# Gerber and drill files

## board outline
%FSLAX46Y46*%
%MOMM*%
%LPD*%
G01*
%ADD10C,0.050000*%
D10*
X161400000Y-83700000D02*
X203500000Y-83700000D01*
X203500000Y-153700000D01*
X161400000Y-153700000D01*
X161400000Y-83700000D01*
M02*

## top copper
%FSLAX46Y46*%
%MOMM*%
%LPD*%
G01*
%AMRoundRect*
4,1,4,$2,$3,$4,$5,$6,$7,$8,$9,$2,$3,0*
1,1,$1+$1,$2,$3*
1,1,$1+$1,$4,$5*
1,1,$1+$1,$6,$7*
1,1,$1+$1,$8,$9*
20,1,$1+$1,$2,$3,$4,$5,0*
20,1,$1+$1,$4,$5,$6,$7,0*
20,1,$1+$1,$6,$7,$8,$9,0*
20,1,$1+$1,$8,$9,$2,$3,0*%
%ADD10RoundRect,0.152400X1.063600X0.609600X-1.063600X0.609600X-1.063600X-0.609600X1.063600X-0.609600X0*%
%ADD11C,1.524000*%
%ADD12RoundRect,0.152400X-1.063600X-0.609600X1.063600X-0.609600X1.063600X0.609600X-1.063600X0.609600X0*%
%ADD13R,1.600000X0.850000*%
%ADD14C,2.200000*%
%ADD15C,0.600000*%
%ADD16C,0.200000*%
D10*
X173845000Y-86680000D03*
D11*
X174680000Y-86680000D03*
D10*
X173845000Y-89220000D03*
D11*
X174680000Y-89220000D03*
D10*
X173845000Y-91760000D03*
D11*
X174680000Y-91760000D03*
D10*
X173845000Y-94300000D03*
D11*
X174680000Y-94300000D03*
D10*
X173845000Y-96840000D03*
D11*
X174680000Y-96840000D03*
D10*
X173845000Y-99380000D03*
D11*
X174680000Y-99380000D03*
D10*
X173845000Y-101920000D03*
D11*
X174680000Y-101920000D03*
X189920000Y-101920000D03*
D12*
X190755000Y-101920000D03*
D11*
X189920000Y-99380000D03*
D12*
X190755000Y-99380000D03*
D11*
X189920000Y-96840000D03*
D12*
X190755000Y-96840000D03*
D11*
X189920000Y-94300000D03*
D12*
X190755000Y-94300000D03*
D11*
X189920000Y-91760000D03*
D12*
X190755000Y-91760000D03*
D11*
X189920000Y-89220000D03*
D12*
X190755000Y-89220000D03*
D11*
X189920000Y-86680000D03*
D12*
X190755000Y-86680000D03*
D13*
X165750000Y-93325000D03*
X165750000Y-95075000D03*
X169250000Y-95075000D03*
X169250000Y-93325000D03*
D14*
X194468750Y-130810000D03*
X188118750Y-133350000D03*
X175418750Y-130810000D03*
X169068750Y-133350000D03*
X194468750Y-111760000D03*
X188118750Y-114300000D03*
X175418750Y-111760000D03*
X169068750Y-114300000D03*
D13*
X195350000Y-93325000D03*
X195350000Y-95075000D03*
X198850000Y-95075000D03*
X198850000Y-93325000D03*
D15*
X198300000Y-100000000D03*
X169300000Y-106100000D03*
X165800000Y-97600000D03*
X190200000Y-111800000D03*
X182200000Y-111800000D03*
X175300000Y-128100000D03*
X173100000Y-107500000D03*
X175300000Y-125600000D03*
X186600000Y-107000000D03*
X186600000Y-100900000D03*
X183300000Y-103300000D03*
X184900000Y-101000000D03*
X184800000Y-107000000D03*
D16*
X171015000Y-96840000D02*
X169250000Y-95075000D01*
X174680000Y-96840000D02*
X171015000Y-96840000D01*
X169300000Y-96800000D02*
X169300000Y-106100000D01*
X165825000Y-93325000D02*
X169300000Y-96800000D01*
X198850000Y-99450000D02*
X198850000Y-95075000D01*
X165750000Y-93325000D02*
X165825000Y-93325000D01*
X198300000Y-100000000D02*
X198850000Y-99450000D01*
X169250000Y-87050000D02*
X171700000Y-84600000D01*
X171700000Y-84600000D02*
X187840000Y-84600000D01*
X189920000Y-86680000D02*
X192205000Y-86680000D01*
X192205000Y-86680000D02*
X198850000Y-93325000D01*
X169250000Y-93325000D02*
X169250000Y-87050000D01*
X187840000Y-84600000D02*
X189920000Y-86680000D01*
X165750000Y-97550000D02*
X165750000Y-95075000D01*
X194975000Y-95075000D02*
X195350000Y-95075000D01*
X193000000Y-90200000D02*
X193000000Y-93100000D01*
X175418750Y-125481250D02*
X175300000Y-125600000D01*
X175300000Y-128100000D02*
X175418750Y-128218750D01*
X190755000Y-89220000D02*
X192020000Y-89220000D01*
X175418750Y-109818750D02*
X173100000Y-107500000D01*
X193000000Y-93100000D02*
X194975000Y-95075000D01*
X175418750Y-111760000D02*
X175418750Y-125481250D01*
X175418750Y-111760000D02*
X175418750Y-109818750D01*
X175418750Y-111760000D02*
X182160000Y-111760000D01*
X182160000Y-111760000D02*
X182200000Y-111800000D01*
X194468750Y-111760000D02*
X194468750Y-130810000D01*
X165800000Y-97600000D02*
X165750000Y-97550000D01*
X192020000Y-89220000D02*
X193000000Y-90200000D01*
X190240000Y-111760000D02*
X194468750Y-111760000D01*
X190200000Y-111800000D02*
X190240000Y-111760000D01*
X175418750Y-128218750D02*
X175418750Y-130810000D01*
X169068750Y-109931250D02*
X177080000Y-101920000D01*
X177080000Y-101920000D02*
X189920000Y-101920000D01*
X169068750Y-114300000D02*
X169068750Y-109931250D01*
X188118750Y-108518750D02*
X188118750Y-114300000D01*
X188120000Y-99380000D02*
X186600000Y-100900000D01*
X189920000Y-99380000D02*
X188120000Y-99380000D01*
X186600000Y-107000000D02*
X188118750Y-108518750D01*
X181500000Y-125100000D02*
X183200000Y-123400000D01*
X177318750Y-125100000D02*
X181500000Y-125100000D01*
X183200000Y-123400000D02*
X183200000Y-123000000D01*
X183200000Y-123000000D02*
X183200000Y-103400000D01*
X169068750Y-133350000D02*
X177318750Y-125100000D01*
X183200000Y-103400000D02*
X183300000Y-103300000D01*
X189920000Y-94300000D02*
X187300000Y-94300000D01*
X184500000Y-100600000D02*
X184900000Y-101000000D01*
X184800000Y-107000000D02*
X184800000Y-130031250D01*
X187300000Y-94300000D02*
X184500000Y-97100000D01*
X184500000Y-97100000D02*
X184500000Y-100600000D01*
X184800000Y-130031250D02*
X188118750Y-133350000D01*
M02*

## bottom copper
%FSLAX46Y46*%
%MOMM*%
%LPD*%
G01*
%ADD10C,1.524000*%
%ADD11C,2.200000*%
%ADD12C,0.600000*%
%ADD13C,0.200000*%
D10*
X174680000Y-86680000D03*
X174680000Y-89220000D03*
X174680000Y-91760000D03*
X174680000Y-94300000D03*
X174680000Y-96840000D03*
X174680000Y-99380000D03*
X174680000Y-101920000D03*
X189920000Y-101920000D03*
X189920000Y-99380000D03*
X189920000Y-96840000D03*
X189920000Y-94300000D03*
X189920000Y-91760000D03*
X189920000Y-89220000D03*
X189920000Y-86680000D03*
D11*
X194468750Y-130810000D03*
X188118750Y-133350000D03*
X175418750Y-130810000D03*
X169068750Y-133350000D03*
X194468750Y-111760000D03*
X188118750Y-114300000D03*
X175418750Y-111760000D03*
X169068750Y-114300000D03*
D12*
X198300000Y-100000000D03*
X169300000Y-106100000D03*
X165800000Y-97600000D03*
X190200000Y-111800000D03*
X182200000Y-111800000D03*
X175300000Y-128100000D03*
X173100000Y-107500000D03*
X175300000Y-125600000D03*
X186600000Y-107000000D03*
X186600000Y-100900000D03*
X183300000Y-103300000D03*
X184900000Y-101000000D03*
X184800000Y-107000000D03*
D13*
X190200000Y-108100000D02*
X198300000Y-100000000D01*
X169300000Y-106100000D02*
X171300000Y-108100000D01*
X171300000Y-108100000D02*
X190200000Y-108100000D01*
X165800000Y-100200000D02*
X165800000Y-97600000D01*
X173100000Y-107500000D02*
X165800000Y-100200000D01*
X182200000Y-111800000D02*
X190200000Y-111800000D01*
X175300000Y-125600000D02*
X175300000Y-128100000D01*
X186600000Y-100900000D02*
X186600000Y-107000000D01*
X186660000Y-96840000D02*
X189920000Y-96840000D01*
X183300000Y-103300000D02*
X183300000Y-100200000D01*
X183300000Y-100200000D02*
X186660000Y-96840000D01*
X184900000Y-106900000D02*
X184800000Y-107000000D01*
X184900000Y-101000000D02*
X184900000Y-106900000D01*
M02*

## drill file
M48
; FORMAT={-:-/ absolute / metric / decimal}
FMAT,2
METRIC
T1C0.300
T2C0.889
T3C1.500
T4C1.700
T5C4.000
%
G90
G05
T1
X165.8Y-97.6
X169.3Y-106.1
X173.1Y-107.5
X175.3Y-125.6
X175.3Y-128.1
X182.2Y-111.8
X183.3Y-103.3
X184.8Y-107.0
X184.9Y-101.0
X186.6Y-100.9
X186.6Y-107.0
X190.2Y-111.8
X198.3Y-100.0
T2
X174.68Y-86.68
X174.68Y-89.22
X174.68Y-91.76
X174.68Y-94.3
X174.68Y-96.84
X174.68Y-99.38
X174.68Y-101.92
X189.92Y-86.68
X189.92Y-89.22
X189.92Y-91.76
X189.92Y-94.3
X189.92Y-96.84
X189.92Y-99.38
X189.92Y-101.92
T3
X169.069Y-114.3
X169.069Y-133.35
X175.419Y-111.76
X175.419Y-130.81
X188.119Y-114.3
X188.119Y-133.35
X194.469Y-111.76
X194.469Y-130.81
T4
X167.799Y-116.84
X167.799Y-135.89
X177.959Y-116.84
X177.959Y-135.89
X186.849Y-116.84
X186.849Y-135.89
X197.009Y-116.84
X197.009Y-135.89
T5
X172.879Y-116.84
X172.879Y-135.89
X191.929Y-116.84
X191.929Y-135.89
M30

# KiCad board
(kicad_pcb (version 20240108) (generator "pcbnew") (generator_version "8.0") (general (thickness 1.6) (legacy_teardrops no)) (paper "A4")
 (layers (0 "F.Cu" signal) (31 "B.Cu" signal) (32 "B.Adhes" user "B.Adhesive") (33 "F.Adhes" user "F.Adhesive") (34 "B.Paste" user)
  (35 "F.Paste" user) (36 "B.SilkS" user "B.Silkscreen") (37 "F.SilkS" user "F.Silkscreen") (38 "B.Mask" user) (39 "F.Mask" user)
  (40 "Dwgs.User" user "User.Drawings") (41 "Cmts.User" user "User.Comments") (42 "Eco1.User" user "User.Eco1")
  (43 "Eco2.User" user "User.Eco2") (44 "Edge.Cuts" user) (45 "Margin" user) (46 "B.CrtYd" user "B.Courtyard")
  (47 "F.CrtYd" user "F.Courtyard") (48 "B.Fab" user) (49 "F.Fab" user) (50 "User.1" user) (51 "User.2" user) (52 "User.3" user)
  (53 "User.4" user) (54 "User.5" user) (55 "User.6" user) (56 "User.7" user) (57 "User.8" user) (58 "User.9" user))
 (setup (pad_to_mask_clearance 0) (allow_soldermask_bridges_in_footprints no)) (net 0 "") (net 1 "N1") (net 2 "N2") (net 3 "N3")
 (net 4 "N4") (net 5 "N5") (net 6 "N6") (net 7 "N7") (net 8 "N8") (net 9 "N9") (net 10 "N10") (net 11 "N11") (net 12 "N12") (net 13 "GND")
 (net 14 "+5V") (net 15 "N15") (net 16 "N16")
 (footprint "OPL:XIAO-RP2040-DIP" (layer "F.Cu") (at 182.3 94.3)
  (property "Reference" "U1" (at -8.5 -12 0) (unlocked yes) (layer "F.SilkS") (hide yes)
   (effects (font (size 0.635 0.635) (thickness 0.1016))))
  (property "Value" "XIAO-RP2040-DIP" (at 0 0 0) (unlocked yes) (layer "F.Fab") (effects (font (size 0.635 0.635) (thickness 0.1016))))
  (pad "1" smd roundrect (at -8.455 -7.62 180) (size 2.432 1.524) (layers "F.Cu" "F.Mask") (roundrect_rratio 0.1) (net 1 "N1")
   (thermal_bridge_angle 45))
  (pad "1" thru_hole circle (at -7.62 -7.62 180) (size 1.524 1.524) (drill 0.889) (layers "*.Cu" "*.Mask") (remove_unused_layers no)
   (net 1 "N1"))
  (pad "2" smd roundrect (at -8.455 -5.08 180) (size 2.432 1.524) (layers "F.Cu" "F.Mask") (roundrect_rratio 0.1) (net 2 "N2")
   (thermal_bridge_angle 45))
  (pad "2" thru_hole circle (at -7.62 -5.08 180) (size 1.524 1.524) (drill 0.889) (layers "*.Cu" "*.Mask") (remove_unused_layers no)
   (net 2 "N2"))
  (pad "3" smd roundrect (at -8.455 -2.54 180) (size 2.432 1.524) (layers "F.Cu" "F.Mask") (roundrect_rratio 0.1) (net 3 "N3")
   (thermal_bridge_angle 45))
  (pad "3" thru_hole circle (at -7.62 -2.54 180) (size 1.524 1.524) (drill 0.889) (layers "*.Cu" "*.Mask") (remove_unused_layers no)
   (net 3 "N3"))
  (pad "4" smd roundrect (at -8.455 0 180) (size 2.432 1.524) (layers "F.Cu" "F.Mask") (roundrect_rratio 0.1) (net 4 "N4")
   (thermal_bridge_angle 45))
  (pad "4" thru_hole circle (at -7.62 0 180) (size 1.524 1.524) (drill 0.889) (layers "*.Cu" "*.Mask") (remove_unused_layers no)
   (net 4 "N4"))
  (pad "5" smd roundrect (at -8.455 2.54 180) (size 2.432 1.524) (layers "F.Cu" "F.Mask") (roundrect_rratio 0.1) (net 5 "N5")
   (thermal_bridge_angle 45))
  (pad "5" thru_hole circle (at -7.62 2.54 180) (size 1.524 1.524) (drill 0.889) (layers "*.Cu" "*.Mask") (remove_unused_layers no)
   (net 5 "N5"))
  (pad "6" smd roundrect (at -8.455 5.08 180) (size 2.432 1.524) (layers "F.Cu" "F.Mask") (roundrect_rratio 0.1) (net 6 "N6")
   (thermal_bridge_angle 45))
  (pad "6" thru_hole circle (at -7.62 5.08 180) (size 1.524 1.524) (drill 0.889) (layers "*.Cu" "*.Mask") (remove_unused_layers no)
   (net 6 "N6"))
  (pad "7" smd roundrect (at -8.455 7.62 180) (size 2.432 1.524) (layers "F.Cu" "F.Mask") (roundrect_rratio 0.1) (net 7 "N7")
   (thermal_bridge_angle 45))
  (pad "7" thru_hole circle (at -7.62 7.62 180) (size 1.524 1.524) (drill 0.889) (layers "*.Cu" "*.Mask") (remove_unused_layers no)
   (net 7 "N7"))
  (pad "8" thru_hole circle (at 7.62 7.62) (size 1.524 1.524) (drill 0.889) (layers "*.Cu" "*.Mask") (remove_unused_layers no) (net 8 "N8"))
  (pad "8" smd roundrect (at 8.455 7.62) (size 2.432 1.524) (layers "F.Cu" "F.Mask") (roundrect_rratio 0.1) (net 8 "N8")
   (thermal_bridge_angle 45))
  (pad "9" thru_hole circle (at 7.62 5.08) (size 1.524 1.524) (drill 0.889) (layers "*.Cu" "*.Mask") (remove_unused_layers no) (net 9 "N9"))
  (pad "9" smd roundrect (at 8.455 5.08) (size 2.432 1.524) (layers "F.Cu" "F.Mask") (roundrect_rratio 0.1) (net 9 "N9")
   (thermal_bridge_angle 45))
  (pad "10" thru_hole circle (at 7.62 2.54) (size 1.524 1.524) (drill 0.889) (layers "*.Cu" "*.Mask") (remove_unused_layers no)
   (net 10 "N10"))
  (pad "10" smd roundrect (at 8.455 2.54) (size 2.432 1.524) (layers "F.Cu" "F.Mask") (roundrect_rratio 0.1) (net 10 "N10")
   (thermal_bridge_angle 45))
  (pad "11" thru_hole circle (at 7.62 0) (size 1.524 1.524) (drill 0.889) (layers "*.Cu" "*.Mask") (remove_unused_layers no) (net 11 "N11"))
  (pad "11" smd roundrect (at 8.455 0) (size 2.432 1.524) (layers "F.Cu" "F.Mask") (roundrect_rratio 0.1) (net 11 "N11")
   (thermal_bridge_angle 45))
  (pad "12" thru_hole circle (at 7.62 -2.54) (size 1.524 1.524) (drill 0.889) (layers "*.Cu" "*.Mask") (remove_unused_layers no)
   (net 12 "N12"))
  (pad "12" smd roundrect (at 8.455 -2.54) (size 2.432 1.524) (layers "F.Cu" "F.Mask") (roundrect_rratio 0.1) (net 12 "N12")
   (thermal_bridge_angle 45))
  (pad "13" thru_hole circle (at 7.62 -5.08) (size 1.524 1.524) (drill 0.889) (layers "*.Cu" "*.Mask") (remove_unused_layers no)
   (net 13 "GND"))
  (pad "13" smd roundrect (at 8.455 -5.08) (size 2.432 1.524) (layers "F.Cu" "F.Mask") (roundrect_rratio 0.1) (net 13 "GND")
   (thermal_bridge_angle 45))
  (pad "14" thru_hole circle (at 7.62 -7.62) (size 1.524 1.524) (drill 0.889) (layers "*.Cu" "*.Mask") (remove_unused_layers no)
   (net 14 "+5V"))
  (pad "14" smd roundrect (at 8.455 -7.62) (size 2.432 1.524) (layers "F.Cu" "F.Mask") (roundrect_rratio 0.1) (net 14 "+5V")
   (thermal_bridge_angle 45)))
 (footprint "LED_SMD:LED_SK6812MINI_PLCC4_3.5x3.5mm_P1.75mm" (layer "F.Cu") (at 167.5 94.2)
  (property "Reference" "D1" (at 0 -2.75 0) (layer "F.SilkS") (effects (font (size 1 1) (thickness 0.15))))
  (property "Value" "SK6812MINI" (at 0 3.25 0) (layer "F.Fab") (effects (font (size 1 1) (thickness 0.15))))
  (pad "1" smd rect (at -1.75 -0.875) (size 1.6 0.85) (layers "F.Cu" "F.Paste" "F.Mask") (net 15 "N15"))
  (pad "2" smd rect (at -1.75 0.875) (size 1.6 0.85) (layers "F.Cu" "F.Paste" "F.Mask") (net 13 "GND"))
  (pad "3" smd rect (at 1.75 0.875) (size 1.6 0.85) (layers "F.Cu" "F.Paste" "F.Mask") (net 5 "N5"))
  (pad "4" smd rect (at 1.75 -0.875) (size 1.6 0.85) (layers "F.Cu" "F.Paste" "F.Mask") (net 14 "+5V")))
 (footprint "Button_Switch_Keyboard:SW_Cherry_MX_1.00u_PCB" (layer "F.Cu") (at 194.46875 130.81)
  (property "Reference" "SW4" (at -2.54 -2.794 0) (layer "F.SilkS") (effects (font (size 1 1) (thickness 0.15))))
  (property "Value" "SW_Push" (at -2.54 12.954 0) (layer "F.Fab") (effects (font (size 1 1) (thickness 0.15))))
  (pad "" np_thru_hole circle (at -7.62 5.08) (size 1.7 1.7) (drill 1.7) (layers "*.Cu" "*.Mask"))
  (pad "" np_thru_hole circle (at -2.54 5.08) (size 4 4) (drill 4) (layers "*.Cu" "*.Mask"))
  (pad "" np_thru_hole circle (at 2.54 5.08) (size 1.7 1.7) (drill 1.7) (layers "*.Cu" "*.Mask"))
  (pad "1" thru_hole circle (at 0 0) (size 2.2 2.2) (drill 1.5) (layers "*.Cu" "*.Mask") (remove_unused_layers no) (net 13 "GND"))
  (pad "2" thru_hole circle (at -6.35 2.54) (size 2.2 2.2) (drill 1.5) (layers "*.Cu" "*.Mask") (remove_unused_layers no) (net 11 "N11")))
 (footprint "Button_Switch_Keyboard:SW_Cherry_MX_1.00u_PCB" (layer "F.Cu") (at 175.41875 130.81)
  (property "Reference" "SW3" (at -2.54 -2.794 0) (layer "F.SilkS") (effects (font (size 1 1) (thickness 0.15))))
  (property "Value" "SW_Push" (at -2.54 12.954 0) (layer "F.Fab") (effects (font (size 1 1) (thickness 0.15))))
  (pad "" np_thru_hole circle (at -7.62 5.08) (size 1.7 1.7) (drill 1.7) (layers "*.Cu" "*.Mask"))
  (pad "" np_thru_hole circle (at -2.54 5.08) (size 4 4) (drill 4) (layers "*.Cu" "*.Mask"))
  (pad "" np_thru_hole circle (at 2.54 5.08) (size 1.7 1.7) (drill 1.7) (layers "*.Cu" "*.Mask"))
  (pad "1" thru_hole circle (at 0 0) (size 2.2 2.2) (drill 1.5) (layers "*.Cu" "*.Mask") (remove_unused_layers no) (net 13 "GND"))
  (pad "2" thru_hole circle (at -6.35 2.54) (size 2.2 2.2) (drill 1.5) (layers "*.Cu" "*.Mask") (remove_unused_layers no) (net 10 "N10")))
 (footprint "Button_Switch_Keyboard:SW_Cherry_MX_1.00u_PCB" (layer "F.Cu") (at 194.46875 111.76)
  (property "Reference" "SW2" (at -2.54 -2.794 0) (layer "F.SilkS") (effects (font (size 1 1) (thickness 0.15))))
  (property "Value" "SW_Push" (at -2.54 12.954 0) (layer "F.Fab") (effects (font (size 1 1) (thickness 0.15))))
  (pad "" np_thru_hole circle (at -7.62 5.08) (size 1.7 1.7) (drill 1.7) (layers "*.Cu" "*.Mask"))
  (pad "" np_thru_hole circle (at -2.54 5.08) (size 4 4) (drill 4) (layers "*.Cu" "*.Mask"))
  (pad "" np_thru_hole circle (at 2.54 5.08) (size 1.7 1.7) (drill 1.7) (layers "*.Cu" "*.Mask"))
  (pad "1" thru_hole circle (at 0 0) (size 2.2 2.2) (drill 1.5) (layers "*.Cu" "*.Mask") (remove_unused_layers no) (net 13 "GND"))
  (pad "2" thru_hole circle (at -6.35 2.54) (size 2.2 2.2) (drill 1.5) (layers "*.Cu" "*.Mask") (remove_unused_layers no) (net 9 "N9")))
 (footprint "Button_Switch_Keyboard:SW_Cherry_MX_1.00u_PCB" (layer "F.Cu") (at 175.41875 111.76)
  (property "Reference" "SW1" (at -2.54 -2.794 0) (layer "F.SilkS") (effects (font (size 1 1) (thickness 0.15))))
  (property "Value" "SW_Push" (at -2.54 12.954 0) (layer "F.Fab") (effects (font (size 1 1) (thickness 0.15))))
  (pad "" np_thru_hole circle (at -7.62 5.08) (size 1.7 1.7) (drill 1.7) (layers "*.Cu" "*.Mask"))
  (pad "" np_thru_hole circle (at -2.54 5.08) (size 4 4) (drill 4) (layers "*.Cu" "*.Mask"))
  (pad "" np_thru_hole circle (at 2.54 5.08) (size 1.7 1.7) (drill 1.7) (layers "*.Cu" "*.Mask"))
  (pad "1" thru_hole circle (at 0 0) (size 2.2 2.2) (drill 1.5) (layers "*.Cu" "*.Mask") (remove_unused_layers no) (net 13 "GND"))
  (pad "2" thru_hole circle (at -6.35 2.54) (size 2.2 2.2) (drill 1.5) (layers "*.Cu" "*.Mask") (remove_unused_layers no) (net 8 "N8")))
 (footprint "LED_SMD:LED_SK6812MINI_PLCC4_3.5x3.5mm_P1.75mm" (layer "F.Cu") (at 197.1 94.2)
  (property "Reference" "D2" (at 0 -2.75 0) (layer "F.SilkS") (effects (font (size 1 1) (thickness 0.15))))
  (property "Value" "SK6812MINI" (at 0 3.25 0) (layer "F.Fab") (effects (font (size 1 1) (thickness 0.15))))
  (pad "1" smd rect (at -1.75 -0.875) (size 1.6 0.85) (layers "F.Cu" "F.Paste" "F.Mask") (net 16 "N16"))
  (pad "2" smd rect (at -1.75 0.875) (size 1.6 0.85) (layers "F.Cu" "F.Paste" "F.Mask") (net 13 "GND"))
  (pad "3" smd rect (at 1.75 0.875) (size 1.6 0.85) (layers "F.Cu" "F.Paste" "F.Mask") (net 15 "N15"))
  (pad "4" smd rect (at 1.75 -0.875) (size 1.6 0.85) (layers "F.Cu" "F.Paste" "F.Mask") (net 14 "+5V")))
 (gr_rect (start 161.4 83.7) (end 203.5 153.7) (stroke (width 0.05) (type default)) (fill none) (layer "Edge.Cuts"))
 (segment (start 171.015 96.84) (end 169.25 95.075) (width 0.2) (layer "F.Cu") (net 5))
 (segment (start 174.68 96.84) (end 171.015 96.84) (width 0.2) (layer "F.Cu") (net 5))
 (segment (start 169.3 96.8) (end 169.3 106.1) (width 0.2) (layer "F.Cu") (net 15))
 (segment (start 165.825 93.325) (end 169.3 96.8) (width 0.2) (layer "F.Cu") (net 15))
 (segment (start 198.85 99.45) (end 198.85 95.075) (width 0.2) (layer "F.Cu") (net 15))
 (segment (start 165.75 93.325) (end 165.825 93.325) (width 0.2) (layer "F.Cu") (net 15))
 (segment (start 198.3 100) (end 198.85 99.45) (width 0.2) (layer "F.Cu") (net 15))
 (via (at 198.3 100) (size 0.6) (drill 0.3) (layers "F.Cu" "B.Cu") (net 15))
 (via (at 169.3 106.1) (size 0.6) (drill 0.3) (layers "F.Cu" "B.Cu") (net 15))
 (segment (start 190.2 108.1) (end 198.3 100) (width 0.2) (layer "B.Cu") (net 15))
 (segment (start 169.3 106.1) (end 171.3 108.1) (width 0.2) (layer "B.Cu") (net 15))
 (segment (start 171.3 108.1) (end 190.2 108.1) (width 0.2) (layer "B.Cu") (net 15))
 (segment (start 169.25 87.05) (end 171.7 84.6) (width 0.2) (layer "F.Cu") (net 14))
 (segment (start 171.7 84.6) (end 187.84 84.6) (width 0.2) (layer "F.Cu") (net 14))
 (segment (start 189.92 86.68) (end 192.205 86.68) (width 0.2) (layer "F.Cu") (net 14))
 (segment (start 192.205 86.68) (end 198.85 93.325) (width 0.2) (layer "F.Cu") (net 14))
 (segment (start 169.25 93.325) (end 169.25 87.05) (width 0.2) (layer "F.Cu") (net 14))
 (segment (start 187.84 84.6) (end 189.92 86.68) (width 0.2) (layer "F.Cu") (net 14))
 (segment (start 165.75 97.55) (end 165.75 95.075) (width 0.2) (layer "F.Cu") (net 13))
 (segment (start 194.975 95.075) (end 195.35 95.075) (width 0.2) (layer "F.Cu") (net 13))
 (segment (start 193 90.2) (end 193 93.1) (width 0.2) (layer "F.Cu") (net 13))
 (segment (start 175.41875 125.48125) (end 175.3 125.6) (width 0.2) (layer "F.Cu") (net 13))
 (segment (start 175.3 128.1) (end 175.41875 128.21875) (width 0.2) (layer "F.Cu") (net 13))
 (segment (start 190.755 89.22) (end 192.02 89.22) (width 0.2) (layer "F.Cu") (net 13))
 (segment (start 175.41875 109.81875) (end 173.1 107.5) (width 0.2) (layer "F.Cu") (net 13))
 (segment (start 193 93.1) (end 194.975 95.075) (width 0.2) (layer "F.Cu") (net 13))
 (segment (start 175.41875 111.76) (end 175.41875 125.48125) (width 0.2) (layer "F.Cu") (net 13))
 (segment (start 175.41875 111.76) (end 175.41875 109.81875) (width 0.2) (layer "F.Cu") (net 13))
 (segment (start 175.41875 111.76) (end 182.16 111.76) (width 0.2) (layer "F.Cu") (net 13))
 (segment (start 182.16 111.76) (end 182.2 111.8) (width 0.2) (layer "F.Cu") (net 13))
 (segment (start 194.46875 111.76) (end 194.46875 130.81) (width 0.2) (layer "F.Cu") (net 13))
 (segment (start 165.8 97.6) (end 165.75 97.55) (width 0.2) (layer "F.Cu") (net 13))
 (segment (start 192.02 89.22) (end 193 90.2) (width 0.2) (layer "F.Cu") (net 13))
 (segment (start 190.24 111.76) (end 194.46875 111.76) (width 0.2) (layer "F.Cu") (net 13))
 (segment (start 190.2 111.8) (end 190.24 111.76) (width 0.2) (layer "F.Cu") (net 13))
 (segment (start 175.41875 128.21875) (end 175.41875 130.81) (width 0.2) (layer "F.Cu") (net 13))
 (via (at 165.8 97.6) (size 0.6) (drill 0.3) (layers "F.Cu" "B.Cu") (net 13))
 (via (at 190.2 111.8) (size 0.6) (drill 0.3) (layers "F.Cu" "B.Cu") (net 13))
 (via (at 182.2 111.8) (size 0.6) (drill 0.3) (layers "F.Cu" "B.Cu") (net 13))
 (via (at 175.3 128.1) (size 0.6) (drill 0.3) (layers "F.Cu" "B.Cu") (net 13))
 (via (at 173.1 107.5) (size 0.6) (drill 0.3) (layers "F.Cu" "B.Cu") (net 13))
 (via (at 175.3 125.6) (size 0.6) (drill 0.3) (layers "F.Cu" "B.Cu") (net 13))
 (segment (start 165.8 100.2) (end 165.8 97.6) (width 0.2) (layer "B.Cu") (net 13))
 (segment (start 173.1 107.5) (end 165.8 100.2) (width 0.2) (layer "B.Cu") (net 13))
 (segment (start 182.2 111.8) (end 190.2 111.8) (width 0.2) (layer "B.Cu") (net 13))
 (segment (start 175.3 125.6) (end 175.3 128.1) (width 0.2) (layer "B.Cu") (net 13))
 (segment (start 169.06875 109.93125) (end 177.08 101.92) (width 0.2) (layer "F.Cu") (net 8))
 (segment (start 177.08 101.92) (end 189.92 101.92) (width 0.2) (layer "F.Cu") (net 8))
 (segment (start 169.06875 114.3) (end 169.06875 109.93125) (width 0.2) (layer "F.Cu") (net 8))
 (segment (start 188.11875 108.51875) (end 188.11875 114.3) (width 0.2) (layer "F.Cu") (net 9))
 (segment (start 188.12 99.38) (end 186.6 100.9) (width 0.2) (layer "F.Cu") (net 9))
 (segment (start 189.92 99.38) (end 188.12 99.38) (width 0.2) (layer "F.Cu") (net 9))
 (segment (start 186.6 107) (end 188.11875 108.51875) (width 0.2) (layer "F.Cu") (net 9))
 (via (at 186.6 107) (size 0.6) (drill 0.3) (layers "F.Cu" "B.Cu") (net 9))
 (via (at 186.6 100.9) (size 0.6) (drill 0.3) (layers "F.Cu" "B.Cu") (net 9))
 (segment (start 186.6 100.9) (end 186.6 107) (width 0.2) (layer "B.Cu") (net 9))
 (segment (start 181.5 125.1) (end 183.2 123.4) (width 0.2) (layer "F.Cu") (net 10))
 (segment (start 177.31875 125.1) (end 181.5 125.1) (width 0.2) (layer "F.Cu") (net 10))
 (segment (start 183.2 123.4) (end 183.2 123) (width 0.2) (layer "F.Cu") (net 10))
 (segment (start 183.2 123) (end 183.2 103.4) (width 0.2) (layer "F.Cu") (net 10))
 (segment (start 169.06875 133.35) (end 177.31875 125.1) (width 0.2) (layer "F.Cu") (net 10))
 (segment (start 183.2 103.4) (end 183.3 103.3) (width 0.2) (layer "F.Cu") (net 10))
 (via (at 183.3 103.3) (size 0.6) (drill 0.3) (layers "F.Cu" "B.Cu") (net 10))
 (segment (start 186.66 96.84) (end 189.92 96.84) (width 0.2) (layer "B.Cu") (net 10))
 (segment (start 183.3 103.3) (end 183.3 100.2) (width 0.2) (layer "B.Cu") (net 10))
 (segment (start 183.3 100.2) (end 186.66 96.84) (width 0.2) (layer "B.Cu") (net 10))
 (segment (start 189.92 94.3) (end 187.3 94.3) (width 0.2) (layer "F.Cu") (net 11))
 (segment (start 184.5 100.6) (end 184.9 101) (width 0.2) (layer "F.Cu") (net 11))
 (segment (start 184.8 107) (end 184.8 130.03125) (width 0.2) (layer "F.Cu") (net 11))
 (segment (start 187.3 94.3) (end 184.5 97.1) (width 0.2) (layer "F.Cu") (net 11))
 (segment (start 184.5 97.1) (end 184.5 100.6) (width 0.2) (layer "F.Cu") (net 11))
 (segment (start 184.8 130.03125) (end 188.11875 133.35) (width 0.2) (layer "F.Cu") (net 11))
 (via (at 184.9 101) (size 0.6) (drill 0.3) (layers "F.Cu" "B.Cu") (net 11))
 (via (at 184.8 107) (size 0.6) (drill 0.3) (layers "F.Cu" "B.Cu") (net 11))
 (segment (start 184.9 106.9) (end 184.8 107) (width 0.2) (layer "B.Cu") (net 11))
 (segment (start 184.9 101) (end 184.9 106.9) (width 0.2) (layer "B.Cu") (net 11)))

